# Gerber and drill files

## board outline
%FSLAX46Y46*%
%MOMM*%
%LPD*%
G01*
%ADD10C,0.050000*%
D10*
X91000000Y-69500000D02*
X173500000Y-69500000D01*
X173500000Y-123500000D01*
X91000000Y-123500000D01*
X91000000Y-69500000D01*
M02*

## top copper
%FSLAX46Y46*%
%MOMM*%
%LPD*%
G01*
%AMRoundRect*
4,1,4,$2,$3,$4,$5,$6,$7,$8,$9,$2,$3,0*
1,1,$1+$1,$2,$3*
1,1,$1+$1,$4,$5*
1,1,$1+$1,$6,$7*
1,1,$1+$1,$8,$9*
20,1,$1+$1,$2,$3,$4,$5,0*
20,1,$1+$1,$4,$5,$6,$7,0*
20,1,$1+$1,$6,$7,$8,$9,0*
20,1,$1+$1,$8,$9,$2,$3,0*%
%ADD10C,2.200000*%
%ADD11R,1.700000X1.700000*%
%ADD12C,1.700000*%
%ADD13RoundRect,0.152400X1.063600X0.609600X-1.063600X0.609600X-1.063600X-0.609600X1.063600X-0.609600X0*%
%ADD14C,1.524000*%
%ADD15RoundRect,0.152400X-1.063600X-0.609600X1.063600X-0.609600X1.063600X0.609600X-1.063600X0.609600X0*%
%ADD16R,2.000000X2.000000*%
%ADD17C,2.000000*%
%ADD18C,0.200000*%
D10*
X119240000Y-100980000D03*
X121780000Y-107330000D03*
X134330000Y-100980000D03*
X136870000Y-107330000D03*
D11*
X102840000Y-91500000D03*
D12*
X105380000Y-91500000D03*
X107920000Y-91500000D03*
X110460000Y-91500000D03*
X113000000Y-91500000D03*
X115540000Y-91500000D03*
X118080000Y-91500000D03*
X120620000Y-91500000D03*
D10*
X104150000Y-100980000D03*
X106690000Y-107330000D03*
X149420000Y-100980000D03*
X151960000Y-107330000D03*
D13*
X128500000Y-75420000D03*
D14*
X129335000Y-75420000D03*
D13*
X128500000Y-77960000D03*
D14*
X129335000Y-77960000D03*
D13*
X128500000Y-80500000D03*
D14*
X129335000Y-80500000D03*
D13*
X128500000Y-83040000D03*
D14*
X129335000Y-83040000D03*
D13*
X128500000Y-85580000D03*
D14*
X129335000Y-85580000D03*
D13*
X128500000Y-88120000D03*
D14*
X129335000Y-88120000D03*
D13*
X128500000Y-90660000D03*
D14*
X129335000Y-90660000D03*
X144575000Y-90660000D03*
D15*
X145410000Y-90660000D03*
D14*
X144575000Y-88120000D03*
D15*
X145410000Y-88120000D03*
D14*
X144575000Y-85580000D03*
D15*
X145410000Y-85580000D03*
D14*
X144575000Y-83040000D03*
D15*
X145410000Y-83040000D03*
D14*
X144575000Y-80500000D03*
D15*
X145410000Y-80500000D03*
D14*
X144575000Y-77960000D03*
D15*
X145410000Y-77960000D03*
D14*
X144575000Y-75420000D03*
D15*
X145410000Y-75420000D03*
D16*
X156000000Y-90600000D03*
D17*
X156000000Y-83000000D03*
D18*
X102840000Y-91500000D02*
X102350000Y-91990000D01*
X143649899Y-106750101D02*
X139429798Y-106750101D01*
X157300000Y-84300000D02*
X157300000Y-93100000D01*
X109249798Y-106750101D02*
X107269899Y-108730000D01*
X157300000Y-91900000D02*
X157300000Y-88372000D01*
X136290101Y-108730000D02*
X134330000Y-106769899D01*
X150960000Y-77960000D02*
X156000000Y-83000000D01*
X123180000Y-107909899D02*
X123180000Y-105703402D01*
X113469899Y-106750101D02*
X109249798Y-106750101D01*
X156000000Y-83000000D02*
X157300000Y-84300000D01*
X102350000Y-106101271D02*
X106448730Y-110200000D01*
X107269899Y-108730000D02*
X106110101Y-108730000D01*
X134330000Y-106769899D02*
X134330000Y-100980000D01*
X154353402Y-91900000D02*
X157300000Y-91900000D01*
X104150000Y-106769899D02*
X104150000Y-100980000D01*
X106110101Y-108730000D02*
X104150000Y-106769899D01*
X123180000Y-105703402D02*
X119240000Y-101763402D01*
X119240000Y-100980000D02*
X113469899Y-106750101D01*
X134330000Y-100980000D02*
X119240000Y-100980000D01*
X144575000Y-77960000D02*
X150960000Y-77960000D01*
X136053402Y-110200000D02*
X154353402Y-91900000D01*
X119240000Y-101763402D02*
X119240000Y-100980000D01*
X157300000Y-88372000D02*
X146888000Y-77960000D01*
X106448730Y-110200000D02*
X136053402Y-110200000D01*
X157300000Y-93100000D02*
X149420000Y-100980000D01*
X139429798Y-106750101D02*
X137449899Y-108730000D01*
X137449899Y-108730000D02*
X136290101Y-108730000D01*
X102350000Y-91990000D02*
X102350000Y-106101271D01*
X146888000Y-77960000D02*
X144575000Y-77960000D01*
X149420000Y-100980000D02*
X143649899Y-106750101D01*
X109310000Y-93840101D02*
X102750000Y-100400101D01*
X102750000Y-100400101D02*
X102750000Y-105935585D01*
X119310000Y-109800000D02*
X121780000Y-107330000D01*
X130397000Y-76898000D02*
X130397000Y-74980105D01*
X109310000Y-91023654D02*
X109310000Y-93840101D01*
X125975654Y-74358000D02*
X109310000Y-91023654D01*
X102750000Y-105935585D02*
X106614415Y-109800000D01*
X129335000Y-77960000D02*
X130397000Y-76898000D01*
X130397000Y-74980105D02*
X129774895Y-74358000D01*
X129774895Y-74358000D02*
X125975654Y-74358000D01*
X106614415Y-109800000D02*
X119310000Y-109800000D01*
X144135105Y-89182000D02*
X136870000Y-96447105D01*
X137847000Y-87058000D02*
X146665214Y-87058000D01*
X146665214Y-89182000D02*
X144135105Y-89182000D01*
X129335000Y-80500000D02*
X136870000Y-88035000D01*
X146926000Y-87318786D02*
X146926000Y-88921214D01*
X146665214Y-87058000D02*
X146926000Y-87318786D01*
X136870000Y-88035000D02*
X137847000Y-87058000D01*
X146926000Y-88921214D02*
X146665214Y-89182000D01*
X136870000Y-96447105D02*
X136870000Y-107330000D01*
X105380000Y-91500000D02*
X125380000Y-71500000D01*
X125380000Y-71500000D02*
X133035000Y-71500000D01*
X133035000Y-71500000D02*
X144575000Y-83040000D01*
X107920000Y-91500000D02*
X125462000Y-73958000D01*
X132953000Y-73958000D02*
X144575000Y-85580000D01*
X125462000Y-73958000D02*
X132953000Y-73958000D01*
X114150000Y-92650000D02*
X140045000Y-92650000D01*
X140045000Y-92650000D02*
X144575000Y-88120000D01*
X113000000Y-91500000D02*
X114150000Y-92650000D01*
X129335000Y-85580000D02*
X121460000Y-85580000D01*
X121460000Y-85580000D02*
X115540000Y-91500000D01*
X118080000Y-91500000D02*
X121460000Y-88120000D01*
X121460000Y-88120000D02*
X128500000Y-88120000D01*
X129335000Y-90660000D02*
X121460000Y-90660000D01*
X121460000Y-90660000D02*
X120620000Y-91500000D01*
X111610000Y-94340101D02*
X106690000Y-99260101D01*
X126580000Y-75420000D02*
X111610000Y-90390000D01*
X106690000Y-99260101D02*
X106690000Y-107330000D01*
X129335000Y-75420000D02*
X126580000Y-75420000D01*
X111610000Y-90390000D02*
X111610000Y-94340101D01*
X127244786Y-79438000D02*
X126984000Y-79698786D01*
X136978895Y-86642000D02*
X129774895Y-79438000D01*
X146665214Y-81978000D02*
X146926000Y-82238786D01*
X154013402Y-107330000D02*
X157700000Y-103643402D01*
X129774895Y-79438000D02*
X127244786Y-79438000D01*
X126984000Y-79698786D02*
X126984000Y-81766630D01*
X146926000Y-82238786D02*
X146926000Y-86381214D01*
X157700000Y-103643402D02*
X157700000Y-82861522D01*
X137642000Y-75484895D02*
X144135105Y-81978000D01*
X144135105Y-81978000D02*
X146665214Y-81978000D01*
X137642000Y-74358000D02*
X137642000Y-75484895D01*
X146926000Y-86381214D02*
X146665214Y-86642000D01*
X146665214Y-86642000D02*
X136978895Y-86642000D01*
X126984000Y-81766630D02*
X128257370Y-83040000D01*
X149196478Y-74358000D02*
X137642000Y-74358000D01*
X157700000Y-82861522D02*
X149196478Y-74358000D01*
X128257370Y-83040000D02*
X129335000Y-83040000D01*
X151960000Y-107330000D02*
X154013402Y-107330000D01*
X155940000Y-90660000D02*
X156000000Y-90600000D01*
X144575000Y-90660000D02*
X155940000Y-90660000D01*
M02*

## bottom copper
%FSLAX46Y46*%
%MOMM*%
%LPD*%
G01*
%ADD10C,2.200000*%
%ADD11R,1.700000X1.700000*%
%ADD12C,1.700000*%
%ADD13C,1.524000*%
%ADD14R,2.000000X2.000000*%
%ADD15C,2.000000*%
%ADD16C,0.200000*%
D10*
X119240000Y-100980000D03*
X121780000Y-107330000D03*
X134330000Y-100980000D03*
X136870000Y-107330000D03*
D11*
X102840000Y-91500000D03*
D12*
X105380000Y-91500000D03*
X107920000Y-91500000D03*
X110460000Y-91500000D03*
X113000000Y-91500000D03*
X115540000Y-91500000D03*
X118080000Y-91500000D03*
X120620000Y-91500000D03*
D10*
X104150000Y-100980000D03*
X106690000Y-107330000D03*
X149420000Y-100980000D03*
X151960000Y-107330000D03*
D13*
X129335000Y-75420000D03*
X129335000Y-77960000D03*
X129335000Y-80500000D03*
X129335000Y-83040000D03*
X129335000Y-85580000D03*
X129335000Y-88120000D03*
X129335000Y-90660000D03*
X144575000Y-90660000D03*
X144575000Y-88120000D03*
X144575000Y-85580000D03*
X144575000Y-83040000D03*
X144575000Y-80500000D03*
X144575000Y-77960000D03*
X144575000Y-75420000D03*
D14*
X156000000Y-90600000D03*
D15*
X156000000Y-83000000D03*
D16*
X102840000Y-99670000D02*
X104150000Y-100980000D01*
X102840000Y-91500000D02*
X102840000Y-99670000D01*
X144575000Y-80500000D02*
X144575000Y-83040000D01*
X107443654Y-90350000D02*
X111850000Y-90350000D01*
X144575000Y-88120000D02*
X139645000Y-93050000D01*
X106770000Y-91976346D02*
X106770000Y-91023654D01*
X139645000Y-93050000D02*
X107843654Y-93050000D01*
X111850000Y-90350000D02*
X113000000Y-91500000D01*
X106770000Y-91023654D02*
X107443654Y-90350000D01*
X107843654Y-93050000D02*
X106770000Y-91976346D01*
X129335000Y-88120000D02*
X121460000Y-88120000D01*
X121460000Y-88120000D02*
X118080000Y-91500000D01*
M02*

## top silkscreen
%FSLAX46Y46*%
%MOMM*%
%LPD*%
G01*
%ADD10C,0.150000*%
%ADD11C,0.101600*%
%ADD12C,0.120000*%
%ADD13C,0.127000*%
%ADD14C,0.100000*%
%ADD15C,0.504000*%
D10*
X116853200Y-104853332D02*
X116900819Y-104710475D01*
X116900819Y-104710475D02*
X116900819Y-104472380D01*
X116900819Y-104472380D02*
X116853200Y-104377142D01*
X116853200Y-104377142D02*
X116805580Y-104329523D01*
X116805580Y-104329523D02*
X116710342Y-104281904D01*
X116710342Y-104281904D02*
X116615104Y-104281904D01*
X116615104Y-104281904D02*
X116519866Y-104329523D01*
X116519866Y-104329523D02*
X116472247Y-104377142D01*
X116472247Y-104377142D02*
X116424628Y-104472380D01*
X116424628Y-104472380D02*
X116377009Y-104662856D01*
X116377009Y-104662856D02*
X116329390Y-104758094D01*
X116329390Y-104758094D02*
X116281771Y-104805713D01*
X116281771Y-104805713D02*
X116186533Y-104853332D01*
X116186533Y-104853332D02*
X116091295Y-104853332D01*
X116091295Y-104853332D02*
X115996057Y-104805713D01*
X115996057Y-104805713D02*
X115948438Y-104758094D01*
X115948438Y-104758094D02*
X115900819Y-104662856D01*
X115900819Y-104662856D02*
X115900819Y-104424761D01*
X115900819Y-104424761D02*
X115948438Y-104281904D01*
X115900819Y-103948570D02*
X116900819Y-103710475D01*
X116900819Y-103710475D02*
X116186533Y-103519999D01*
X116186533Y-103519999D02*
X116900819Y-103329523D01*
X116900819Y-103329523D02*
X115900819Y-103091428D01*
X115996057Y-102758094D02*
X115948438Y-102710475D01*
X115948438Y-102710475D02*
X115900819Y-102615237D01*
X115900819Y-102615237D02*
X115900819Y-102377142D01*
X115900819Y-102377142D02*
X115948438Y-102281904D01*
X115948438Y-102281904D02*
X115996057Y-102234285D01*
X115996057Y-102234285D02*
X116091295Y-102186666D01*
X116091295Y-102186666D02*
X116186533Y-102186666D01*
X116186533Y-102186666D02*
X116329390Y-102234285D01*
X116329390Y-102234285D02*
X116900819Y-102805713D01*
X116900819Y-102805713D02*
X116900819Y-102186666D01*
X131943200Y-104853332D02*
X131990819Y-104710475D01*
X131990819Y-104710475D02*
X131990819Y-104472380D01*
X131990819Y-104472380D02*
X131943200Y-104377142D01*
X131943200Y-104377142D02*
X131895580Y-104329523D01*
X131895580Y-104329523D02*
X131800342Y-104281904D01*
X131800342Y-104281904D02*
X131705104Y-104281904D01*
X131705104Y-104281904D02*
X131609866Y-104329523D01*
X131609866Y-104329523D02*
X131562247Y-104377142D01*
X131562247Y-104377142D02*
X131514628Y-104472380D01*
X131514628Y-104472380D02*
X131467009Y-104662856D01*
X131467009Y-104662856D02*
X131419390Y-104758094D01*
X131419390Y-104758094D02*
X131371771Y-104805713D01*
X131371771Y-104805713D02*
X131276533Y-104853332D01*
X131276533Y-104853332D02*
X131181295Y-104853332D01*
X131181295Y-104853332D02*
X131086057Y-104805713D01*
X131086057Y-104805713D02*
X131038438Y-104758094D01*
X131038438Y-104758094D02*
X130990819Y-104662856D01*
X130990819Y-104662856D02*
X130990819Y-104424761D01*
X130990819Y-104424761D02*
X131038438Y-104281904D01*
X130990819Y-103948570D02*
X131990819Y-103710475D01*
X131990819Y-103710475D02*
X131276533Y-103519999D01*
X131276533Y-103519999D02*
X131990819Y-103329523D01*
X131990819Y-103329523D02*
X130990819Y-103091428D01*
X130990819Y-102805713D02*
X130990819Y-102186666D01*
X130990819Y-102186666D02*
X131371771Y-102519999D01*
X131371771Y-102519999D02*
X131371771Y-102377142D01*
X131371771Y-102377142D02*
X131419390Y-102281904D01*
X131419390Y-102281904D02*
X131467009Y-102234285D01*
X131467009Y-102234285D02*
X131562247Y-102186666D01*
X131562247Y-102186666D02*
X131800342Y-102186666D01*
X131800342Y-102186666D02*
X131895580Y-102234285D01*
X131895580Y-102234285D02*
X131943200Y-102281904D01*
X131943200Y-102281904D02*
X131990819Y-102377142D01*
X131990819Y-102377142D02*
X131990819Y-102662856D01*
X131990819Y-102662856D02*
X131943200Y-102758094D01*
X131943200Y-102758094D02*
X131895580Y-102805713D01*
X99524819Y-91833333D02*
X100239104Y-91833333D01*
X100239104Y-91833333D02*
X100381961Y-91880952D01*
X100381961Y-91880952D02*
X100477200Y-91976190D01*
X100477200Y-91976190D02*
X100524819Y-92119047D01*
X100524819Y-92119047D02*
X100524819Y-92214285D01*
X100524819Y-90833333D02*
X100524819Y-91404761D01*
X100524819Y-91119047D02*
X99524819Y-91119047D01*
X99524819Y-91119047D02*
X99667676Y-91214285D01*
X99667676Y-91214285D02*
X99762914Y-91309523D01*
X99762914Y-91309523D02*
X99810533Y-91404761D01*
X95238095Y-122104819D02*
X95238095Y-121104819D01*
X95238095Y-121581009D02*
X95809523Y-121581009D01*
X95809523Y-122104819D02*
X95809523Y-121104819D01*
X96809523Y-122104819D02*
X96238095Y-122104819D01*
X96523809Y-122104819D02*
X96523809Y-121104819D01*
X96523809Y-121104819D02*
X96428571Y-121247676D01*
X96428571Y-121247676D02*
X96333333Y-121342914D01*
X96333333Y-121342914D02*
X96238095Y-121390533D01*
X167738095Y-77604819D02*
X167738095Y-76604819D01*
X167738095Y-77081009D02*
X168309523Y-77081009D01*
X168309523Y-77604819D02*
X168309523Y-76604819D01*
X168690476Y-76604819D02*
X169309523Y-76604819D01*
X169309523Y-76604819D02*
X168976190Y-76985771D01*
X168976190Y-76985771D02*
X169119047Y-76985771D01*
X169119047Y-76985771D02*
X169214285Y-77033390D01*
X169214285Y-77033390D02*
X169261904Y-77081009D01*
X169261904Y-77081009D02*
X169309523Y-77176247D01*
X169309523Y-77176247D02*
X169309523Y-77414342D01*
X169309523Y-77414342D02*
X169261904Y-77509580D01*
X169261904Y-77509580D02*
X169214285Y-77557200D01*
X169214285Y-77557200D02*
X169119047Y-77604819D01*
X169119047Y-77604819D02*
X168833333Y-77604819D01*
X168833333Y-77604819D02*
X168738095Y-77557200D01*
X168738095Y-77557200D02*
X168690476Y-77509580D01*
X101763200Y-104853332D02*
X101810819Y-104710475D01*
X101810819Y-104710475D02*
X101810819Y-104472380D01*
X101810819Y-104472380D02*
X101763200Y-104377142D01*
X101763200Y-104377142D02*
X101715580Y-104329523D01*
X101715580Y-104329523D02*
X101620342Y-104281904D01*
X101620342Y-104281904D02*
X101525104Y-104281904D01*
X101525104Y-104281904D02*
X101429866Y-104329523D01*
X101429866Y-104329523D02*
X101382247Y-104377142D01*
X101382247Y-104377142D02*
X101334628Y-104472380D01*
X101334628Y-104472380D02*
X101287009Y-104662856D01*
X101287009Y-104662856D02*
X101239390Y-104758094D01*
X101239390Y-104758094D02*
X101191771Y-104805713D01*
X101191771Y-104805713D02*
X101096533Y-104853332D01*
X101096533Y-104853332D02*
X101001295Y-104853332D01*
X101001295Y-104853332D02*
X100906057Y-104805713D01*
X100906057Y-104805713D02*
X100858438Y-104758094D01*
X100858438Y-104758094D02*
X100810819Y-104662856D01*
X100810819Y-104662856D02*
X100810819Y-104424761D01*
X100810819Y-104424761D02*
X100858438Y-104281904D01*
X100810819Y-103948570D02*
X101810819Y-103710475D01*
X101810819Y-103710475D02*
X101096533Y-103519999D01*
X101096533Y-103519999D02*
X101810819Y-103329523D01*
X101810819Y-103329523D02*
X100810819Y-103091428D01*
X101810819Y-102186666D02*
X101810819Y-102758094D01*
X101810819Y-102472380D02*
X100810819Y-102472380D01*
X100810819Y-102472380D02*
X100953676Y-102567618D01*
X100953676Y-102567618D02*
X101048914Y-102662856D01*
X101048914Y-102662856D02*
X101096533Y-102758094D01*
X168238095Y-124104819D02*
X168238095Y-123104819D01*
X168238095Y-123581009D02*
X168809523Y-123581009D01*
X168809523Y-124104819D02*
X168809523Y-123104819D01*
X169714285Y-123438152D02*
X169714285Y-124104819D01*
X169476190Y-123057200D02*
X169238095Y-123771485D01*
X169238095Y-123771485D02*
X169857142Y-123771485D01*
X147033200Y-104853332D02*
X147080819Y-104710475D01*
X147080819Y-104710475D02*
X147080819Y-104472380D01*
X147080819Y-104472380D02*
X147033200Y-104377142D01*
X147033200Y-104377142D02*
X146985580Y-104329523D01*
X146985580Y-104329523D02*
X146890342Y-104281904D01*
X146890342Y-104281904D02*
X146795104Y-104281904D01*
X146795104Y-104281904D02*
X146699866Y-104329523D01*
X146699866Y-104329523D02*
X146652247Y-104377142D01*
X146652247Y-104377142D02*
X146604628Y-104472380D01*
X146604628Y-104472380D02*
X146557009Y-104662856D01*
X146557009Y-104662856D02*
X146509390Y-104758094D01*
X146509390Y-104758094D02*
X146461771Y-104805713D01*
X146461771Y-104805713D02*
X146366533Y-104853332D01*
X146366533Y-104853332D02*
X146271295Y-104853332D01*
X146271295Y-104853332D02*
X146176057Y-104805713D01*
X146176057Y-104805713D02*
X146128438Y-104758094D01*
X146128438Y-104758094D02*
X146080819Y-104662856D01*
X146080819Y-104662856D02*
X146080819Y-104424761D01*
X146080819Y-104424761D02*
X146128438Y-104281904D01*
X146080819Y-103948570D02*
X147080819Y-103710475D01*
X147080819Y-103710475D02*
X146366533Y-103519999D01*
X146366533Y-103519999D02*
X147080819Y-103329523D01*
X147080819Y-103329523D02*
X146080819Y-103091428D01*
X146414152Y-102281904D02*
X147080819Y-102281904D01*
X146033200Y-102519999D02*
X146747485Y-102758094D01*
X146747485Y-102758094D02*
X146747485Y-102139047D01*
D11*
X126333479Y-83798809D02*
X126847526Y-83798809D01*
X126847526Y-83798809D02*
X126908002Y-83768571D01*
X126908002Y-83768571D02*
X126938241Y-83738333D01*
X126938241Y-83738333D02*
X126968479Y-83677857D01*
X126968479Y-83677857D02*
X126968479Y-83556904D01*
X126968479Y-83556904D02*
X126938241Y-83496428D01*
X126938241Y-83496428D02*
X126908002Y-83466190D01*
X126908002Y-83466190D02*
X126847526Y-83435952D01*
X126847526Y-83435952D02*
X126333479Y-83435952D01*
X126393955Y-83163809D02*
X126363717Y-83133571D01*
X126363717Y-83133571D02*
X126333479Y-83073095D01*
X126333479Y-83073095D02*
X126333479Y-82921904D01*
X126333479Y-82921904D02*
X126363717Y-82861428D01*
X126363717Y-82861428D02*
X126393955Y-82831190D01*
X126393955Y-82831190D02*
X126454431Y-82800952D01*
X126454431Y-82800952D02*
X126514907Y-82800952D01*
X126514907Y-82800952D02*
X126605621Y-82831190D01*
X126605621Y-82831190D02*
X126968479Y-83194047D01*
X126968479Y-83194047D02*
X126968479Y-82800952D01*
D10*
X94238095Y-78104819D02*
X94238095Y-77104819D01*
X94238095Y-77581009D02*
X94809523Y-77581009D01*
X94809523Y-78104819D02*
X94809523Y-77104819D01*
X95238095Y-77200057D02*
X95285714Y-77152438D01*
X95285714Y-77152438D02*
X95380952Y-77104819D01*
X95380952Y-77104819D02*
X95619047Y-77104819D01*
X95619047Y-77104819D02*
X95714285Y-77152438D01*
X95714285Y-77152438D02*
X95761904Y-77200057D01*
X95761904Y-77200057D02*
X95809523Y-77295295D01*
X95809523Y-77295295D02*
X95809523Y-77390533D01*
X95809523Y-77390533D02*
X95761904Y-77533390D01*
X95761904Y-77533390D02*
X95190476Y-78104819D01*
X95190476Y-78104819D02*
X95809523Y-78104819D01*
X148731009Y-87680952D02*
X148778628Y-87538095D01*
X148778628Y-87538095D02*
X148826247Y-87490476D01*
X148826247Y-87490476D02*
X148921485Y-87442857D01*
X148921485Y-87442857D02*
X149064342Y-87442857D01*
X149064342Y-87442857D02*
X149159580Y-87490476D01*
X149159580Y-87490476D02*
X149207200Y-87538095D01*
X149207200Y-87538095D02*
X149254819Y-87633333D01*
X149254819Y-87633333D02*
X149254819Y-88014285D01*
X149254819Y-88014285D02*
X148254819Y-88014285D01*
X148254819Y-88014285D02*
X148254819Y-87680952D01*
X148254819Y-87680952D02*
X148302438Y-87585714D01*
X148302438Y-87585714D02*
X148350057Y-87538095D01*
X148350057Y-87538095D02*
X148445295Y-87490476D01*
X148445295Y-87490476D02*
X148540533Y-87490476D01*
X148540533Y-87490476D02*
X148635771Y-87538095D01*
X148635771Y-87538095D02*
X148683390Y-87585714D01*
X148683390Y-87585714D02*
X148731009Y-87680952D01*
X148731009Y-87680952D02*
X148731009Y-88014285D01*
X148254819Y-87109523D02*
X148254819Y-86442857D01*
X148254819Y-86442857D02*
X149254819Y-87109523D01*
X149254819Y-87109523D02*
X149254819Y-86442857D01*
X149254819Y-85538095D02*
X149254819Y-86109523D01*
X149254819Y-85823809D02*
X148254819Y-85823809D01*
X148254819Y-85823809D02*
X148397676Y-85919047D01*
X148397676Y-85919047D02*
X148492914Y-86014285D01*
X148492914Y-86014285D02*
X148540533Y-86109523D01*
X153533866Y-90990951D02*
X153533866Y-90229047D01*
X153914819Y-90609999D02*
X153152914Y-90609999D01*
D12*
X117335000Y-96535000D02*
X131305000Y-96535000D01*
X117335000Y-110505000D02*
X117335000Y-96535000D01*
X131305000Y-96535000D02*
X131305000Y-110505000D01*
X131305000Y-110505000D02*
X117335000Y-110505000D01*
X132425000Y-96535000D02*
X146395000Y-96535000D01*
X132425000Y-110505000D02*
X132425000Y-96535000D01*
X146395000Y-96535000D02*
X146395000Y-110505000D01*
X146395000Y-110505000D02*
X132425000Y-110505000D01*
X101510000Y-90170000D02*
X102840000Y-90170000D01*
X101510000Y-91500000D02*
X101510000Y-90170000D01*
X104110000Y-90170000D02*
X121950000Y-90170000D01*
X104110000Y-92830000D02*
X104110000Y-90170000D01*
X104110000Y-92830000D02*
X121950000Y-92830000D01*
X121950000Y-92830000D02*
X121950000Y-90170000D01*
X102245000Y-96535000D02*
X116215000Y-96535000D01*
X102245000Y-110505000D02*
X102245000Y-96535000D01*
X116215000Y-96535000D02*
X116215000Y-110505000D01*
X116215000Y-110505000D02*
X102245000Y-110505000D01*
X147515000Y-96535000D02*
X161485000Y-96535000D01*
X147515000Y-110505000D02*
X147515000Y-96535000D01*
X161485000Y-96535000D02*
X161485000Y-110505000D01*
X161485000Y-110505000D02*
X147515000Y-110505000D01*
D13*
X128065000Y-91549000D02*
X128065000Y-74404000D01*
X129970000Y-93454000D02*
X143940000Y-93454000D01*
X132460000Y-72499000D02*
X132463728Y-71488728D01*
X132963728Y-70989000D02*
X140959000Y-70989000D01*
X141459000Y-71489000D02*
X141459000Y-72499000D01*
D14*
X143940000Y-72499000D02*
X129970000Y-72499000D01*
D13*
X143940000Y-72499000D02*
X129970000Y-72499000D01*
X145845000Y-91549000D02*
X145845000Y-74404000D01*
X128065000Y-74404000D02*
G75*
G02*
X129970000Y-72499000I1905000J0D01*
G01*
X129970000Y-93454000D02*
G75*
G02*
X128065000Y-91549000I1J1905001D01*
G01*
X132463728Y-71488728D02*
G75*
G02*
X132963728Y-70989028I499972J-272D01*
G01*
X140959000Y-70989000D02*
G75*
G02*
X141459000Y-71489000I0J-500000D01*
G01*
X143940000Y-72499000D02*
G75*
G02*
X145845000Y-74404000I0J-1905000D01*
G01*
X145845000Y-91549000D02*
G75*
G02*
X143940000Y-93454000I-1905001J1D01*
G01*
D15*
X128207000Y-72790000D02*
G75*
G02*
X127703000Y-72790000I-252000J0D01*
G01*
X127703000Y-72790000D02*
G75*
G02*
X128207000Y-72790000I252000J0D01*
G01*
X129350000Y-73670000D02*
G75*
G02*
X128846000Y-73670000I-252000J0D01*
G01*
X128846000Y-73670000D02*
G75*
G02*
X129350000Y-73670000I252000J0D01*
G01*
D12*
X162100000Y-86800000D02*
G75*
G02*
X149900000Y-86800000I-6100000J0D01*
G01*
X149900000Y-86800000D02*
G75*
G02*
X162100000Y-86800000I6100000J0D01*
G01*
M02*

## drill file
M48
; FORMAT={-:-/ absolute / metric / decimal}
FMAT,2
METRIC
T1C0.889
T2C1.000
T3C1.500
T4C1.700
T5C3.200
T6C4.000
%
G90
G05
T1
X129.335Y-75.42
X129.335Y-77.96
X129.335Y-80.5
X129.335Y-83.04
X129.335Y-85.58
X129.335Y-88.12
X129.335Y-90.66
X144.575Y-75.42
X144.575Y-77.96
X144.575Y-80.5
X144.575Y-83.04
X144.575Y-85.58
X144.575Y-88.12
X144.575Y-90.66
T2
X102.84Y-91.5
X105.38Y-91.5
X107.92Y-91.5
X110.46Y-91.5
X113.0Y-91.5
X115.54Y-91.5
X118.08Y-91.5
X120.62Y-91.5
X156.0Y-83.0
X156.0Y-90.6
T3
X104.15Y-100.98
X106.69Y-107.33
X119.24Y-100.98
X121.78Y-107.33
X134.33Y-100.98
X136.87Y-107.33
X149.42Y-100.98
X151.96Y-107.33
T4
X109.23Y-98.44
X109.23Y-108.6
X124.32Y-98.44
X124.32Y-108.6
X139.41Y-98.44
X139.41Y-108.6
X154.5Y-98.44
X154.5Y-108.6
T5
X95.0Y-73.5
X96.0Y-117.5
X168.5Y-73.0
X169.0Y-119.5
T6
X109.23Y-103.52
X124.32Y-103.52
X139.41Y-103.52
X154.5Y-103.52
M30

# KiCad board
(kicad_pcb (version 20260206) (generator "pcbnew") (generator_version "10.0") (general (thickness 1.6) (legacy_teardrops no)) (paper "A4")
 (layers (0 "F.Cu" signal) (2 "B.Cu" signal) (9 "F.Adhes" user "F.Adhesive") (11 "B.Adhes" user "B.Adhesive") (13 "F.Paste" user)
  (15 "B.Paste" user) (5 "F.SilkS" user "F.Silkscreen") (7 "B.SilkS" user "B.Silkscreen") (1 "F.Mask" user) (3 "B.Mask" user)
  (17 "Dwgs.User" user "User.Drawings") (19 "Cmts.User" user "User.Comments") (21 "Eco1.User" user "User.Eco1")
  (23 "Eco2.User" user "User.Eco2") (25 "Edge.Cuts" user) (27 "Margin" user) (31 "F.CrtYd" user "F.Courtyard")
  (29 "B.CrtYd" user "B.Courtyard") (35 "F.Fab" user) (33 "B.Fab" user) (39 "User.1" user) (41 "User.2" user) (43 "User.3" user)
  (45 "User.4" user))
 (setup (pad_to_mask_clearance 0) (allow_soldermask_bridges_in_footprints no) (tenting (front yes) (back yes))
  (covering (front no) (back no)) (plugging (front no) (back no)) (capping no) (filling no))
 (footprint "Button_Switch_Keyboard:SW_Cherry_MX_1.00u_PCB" (layer "F.Cu") (at 119.24 100.98 90)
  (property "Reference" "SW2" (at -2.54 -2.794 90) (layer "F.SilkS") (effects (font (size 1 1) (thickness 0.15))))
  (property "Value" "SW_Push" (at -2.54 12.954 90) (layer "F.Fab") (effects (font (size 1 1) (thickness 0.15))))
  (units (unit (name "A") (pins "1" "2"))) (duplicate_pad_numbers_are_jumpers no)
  (fp_line (start 4.445 -1.905) (end 4.445 12.065) (stroke (width 0.12) (type solid)) (layer "F.SilkS"))
  (fp_line (start -9.525 -1.905) (end 4.445 -1.905) (stroke (width 0.12) (type solid)) (layer "F.SilkS"))
  (fp_line (start 4.445 12.065) (end -9.525 12.065) (stroke (width 0.12) (type solid)) (layer "F.SilkS"))
  (fp_line (start -9.525 12.065) (end -9.525 -1.905) (stroke (width 0.12) (type solid)) (layer "F.SilkS"))
  (pad "" np_thru_hole circle (at -7.62 5.08 90) (size 1.7 1.7) (drill 1.7) (layers "*.Cu" "*.Mask"))
  (pad "" np_thru_hole circle (at -2.54 5.08 90) (size 4 4) (drill 4) (layers "*.Cu" "*.Mask"))
  (pad "" np_thru_hole circle (at 2.54 5.08 90) (size 1.7 1.7) (drill 1.7) (layers "*.Cu" "*.Mask"))
  (pad "1" thru_hole circle (at 0 0 90) (size 2.2 2.2) (drill 1.5) (layers "*.Cu" "*.Mask") (remove_unused_layers no) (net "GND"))
  (pad "2" thru_hole circle (at -6.35 2.54 90) (size 2.2 2.2) (drill 1.5) (layers "*.Cu" "*.Mask") (remove_unused_layers no)
   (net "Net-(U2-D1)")))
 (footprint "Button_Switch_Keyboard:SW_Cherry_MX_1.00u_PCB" (layer "F.Cu") (at 134.33 100.98 90)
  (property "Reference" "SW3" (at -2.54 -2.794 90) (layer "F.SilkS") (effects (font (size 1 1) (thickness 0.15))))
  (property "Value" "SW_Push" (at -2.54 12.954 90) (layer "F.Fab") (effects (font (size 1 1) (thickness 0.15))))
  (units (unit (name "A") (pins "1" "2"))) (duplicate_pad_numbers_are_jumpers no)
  (fp_line (start 4.445 -1.905) (end 4.445 12.065) (stroke (width 0.12) (type solid)) (layer "F.SilkS"))
  (fp_line (start -9.525 -1.905) (end 4.445 -1.905) (stroke (width 0.12) (type solid)) (layer "F.SilkS"))
  (fp_line (start 4.445 12.065) (end -9.525 12.065) (stroke (width 0.12) (type solid)) (layer "F.SilkS"))
  (fp_line (start -9.525 12.065) (end -9.525 -1.905) (stroke (width 0.12) (type solid)) (layer "F.SilkS"))
  (pad "" np_thru_hole circle (at -7.62 5.08 90) (size 1.7 1.7) (drill 1.7) (layers "*.Cu" "*.Mask"))
  (pad "" np_thru_hole circle (at -2.54 5.08 90) (size 4 4) (drill 4) (layers "*.Cu" "*.Mask"))
  (pad "" np_thru_hole circle (at 2.54 5.08 90) (size 1.7 1.7) (drill 1.7) (layers "*.Cu" "*.Mask"))
  (pad "1" thru_hole circle (at 0 0 90) (size 2.2 2.2) (drill 1.5) (layers "*.Cu" "*.Mask") (remove_unused_layers no) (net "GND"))
  (pad "2" thru_hole circle (at -6.35 2.54 90) (size 2.2 2.2) (drill 1.5) (layers "*.Cu" "*.Mask") (remove_unused_layers no)
   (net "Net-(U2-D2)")))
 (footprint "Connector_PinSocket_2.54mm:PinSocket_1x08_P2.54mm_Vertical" (layer "F.Cu") (at 102.84 91.5 90)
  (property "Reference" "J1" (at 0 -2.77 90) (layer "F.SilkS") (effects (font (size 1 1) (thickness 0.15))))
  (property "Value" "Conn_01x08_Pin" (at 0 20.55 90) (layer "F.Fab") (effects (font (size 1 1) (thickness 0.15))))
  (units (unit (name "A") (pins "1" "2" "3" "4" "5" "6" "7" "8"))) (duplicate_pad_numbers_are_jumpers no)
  (fp_line (start 1.33 -1.33) (end 1.33 0) (stroke (width 0.12) (type solid)) (layer "F.SilkS"))
  (fp_line (start 0 -1.33) (end 1.33 -1.33) (stroke (width 0.12) (type solid)) (layer "F.SilkS"))
  (fp_line (start 1.33 1.27) (end 1.33 19.11) (stroke (width 0.12) (type solid)) (layer "F.SilkS"))
  (fp_line (start -1.33 1.27) (end 1.33 1.27) (stroke (width 0.12) (type solid)) (layer "F.SilkS"))
  (fp_line (start -1.33 1.27) (end -1.33 19.11) (stroke (width 0.12) (type solid)) (layer "F.SilkS"))
  (fp_line (start -1.33 19.11) (end 1.33 19.11) (stroke (width 0.12) (type solid)) (layer "F.SilkS"))
  (pad "1" thru_hole rect (at 0 0 90) (size 1.7 1.7) (drill 1) (layers "*.Cu" "*.Mask") (remove_unused_layers no) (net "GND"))
  (pad "2" thru_hole circle (at 0 2.54 90) (size 1.7 1.7) (drill 1) (layers "*.Cu" "*.Mask") (remove_unused_layers no) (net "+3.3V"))
  (pad "3" thru_hole circle (at 0 5.08 90) (size 1.7 1.7) (drill 1) (layers "*.Cu" "*.Mask") (remove_unused_layers no) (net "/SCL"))
  (pad "4" thru_hole circle (at 0 7.62 90) (size 1.7 1.7) (drill 1) (layers "*.Cu" "*.Mask") (remove_unused_layers no) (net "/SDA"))
  (pad "5" thru_hole circle (at 0 10.16 90) (size 1.7 1.7) (drill 1) (layers "*.Cu" "*.Mask") (remove_unused_layers no) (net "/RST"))
  (pad "6" thru_hole circle (at 0 12.7 90) (size 1.7 1.7) (drill 1) (layers "*.Cu" "*.Mask") (remove_unused_layers no) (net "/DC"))
  (pad "7" thru_hole circle (at 0 15.24 90) (size 1.7 1.7) (drill 1) (layers "*.Cu" "*.Mask") (remove_unused_layers no) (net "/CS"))
  (pad "8" thru_hole circle (at 0 17.78 90) (size 1.7 1.7) (drill 1) (layers "*.Cu" "*.Mask") (remove_unused_layers no) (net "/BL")))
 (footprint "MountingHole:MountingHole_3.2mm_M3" (layer "F.Cu") (at 96 117.5 180)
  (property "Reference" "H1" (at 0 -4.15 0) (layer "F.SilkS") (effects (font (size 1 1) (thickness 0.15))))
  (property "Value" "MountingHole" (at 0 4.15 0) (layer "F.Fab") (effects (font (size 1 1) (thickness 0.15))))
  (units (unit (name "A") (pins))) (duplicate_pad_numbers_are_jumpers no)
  (pad "" np_thru_hole circle (at 0 0 180) (size 3.2 3.2) (drill 3.2) (layers "*.Cu" "*.Mask")))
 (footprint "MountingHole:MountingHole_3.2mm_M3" (layer "F.Cu") (at 168.5 73 180)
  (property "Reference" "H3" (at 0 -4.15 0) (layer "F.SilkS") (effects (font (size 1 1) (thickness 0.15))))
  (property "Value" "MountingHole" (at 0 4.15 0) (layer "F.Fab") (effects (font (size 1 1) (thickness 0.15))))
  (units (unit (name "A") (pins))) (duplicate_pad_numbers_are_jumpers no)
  (pad "" np_thru_hole circle (at 0 0 180) (size 3.2 3.2) (drill 3.2) (layers "*.Cu" "*.Mask")))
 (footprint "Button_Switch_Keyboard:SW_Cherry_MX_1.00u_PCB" (layer "F.Cu") (at 104.15 100.98 90)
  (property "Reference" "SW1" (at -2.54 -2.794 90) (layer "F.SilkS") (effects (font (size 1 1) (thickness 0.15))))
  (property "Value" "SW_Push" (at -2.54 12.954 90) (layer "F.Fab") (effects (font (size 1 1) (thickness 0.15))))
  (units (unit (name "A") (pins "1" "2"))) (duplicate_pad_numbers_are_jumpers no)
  (fp_line (start 4.445 -1.905) (end 4.445 12.065) (stroke (width 0.12) (type solid)) (layer "F.SilkS"))
  (fp_line (start -9.525 -1.905) (end 4.445 -1.905) (stroke (width 0.12) (type solid)) (layer "F.SilkS"))
  (fp_line (start 4.445 12.065) (end -9.525 12.065) (stroke (width 0.12) (type solid)) (layer "F.SilkS"))
  (fp_line (start -9.525 12.065) (end -9.525 -1.905) (stroke (width 0.12) (type solid)) (layer "F.SilkS"))
  (pad "" np_thru_hole circle (at -7.62 5.08 90) (size 1.7 1.7) (drill 1.7) (layers "*.Cu" "*.Mask"))
  (pad "" np_thru_hole circle (at -2.54 5.08 90) (size 4 4) (drill 4) (layers "*.Cu" "*.Mask"))
  (pad "" np_thru_hole circle (at 2.54 5.08 90) (size 1.7 1.7) (drill 1.7) (layers "*.Cu" "*.Mask"))
  (pad "1" thru_hole circle (at 0 0 90) (size 2.2 2.2) (drill 1.5) (layers "*.Cu" "*.Mask") (remove_unused_layers no) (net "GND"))
  (pad "2" thru_hole circle (at -6.35 2.54 90) (size 2.2 2.2) (drill 1.5) (layers "*.Cu" "*.Mask") (remove_unused_layers no)
   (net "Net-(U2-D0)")))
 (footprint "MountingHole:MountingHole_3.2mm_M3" (layer "F.Cu") (at 169 119.5 180)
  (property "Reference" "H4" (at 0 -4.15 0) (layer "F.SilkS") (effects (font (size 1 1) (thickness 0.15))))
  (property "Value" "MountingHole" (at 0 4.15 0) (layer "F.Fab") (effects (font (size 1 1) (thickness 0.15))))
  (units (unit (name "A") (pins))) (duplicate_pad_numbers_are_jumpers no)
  (pad "" np_thru_hole circle (at 0 0 180) (size 3.2 3.2) (drill 3.2) (layers "*.Cu" "*.Mask")))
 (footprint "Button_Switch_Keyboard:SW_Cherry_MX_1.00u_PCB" (layer "F.Cu") (at 149.42 100.98 90)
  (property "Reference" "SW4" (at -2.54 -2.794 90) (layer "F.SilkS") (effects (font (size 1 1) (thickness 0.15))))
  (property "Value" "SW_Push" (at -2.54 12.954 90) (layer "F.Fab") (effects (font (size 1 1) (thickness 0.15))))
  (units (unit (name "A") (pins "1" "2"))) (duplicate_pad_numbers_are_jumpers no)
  (fp_line (start 4.445 -1.905) (end 4.445 12.065) (stroke (width 0.12) (type solid)) (layer "F.SilkS"))
  (fp_line (start -9.525 -1.905) (end 4.445 -1.905) (stroke (width 0.12) (type solid)) (layer "F.SilkS"))
  (fp_line (start 4.445 12.065) (end -9.525 12.065) (stroke (width 0.12) (type solid)) (layer "F.SilkS"))
  (fp_line (start -9.525 12.065) (end -9.525 -1.905) (stroke (width 0.12) (type solid)) (layer "F.SilkS"))
  (pad "" np_thru_hole circle (at -7.62 5.08 90) (size 1.7 1.7) (drill 1.7) (layers "*.Cu" "*.Mask"))
  (pad "" np_thru_hole circle (at -2.54 5.08 90) (size 4 4) (drill 4) (layers "*.Cu" "*.Mask"))
  (pad "" np_thru_hole circle (at 2.54 5.08 90) (size 1.7 1.7) (drill 1.7) (layers "*.Cu" "*.Mask"))
  (pad "1" thru_hole circle (at 0 0 90) (size 2.2 2.2) (drill 1.5) (layers "*.Cu" "*.Mask") (remove_unused_layers no) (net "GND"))
  (pad "2" thru_hole circle (at -6.35 2.54 90) (size 2.2 2.2) (drill 1.5) (layers "*.Cu" "*.Mask") (remove_unused_layers no)
   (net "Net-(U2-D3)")))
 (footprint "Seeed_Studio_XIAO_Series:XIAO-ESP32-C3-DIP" (layer "F.Cu") (at 136.955 83.04 90)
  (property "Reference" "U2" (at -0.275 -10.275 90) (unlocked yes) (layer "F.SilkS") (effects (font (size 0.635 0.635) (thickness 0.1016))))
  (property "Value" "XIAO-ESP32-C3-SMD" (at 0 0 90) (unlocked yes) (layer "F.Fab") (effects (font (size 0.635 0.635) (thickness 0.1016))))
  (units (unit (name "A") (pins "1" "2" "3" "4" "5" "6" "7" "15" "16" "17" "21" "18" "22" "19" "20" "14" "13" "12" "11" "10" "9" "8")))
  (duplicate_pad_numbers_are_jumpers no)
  (fp_line (start -8.509 -8.89) (end 8.636 -8.89) (stroke (width 0.127) (type solid)) (layer "F.SilkS"))
  (fp_line (start -10.414 -6.985) (end -10.414 6.985) (stroke (width 0.127) (type solid)) (layer "F.SilkS"))
  (fp_line (start 10.541 -4.495) (end 11.551272 -4.491272) (stroke (width 0.127) (type solid)) (layer "F.SilkS"))
  (fp_line (start 12.051 -3.991272) (end 12.051 4.004) (stroke (width 0.127) (type solid)) (layer "F.SilkS"))
  (fp_line (start 11.551 4.504) (end 10.541 4.504) (stroke (width 0.127) (type solid)) (layer "F.SilkS"))
  (fp_line (start 10.541 6.985) (end 10.541 -6.985) (stroke (width 0.1) (type solid)) (layer "F.SilkS"))
  (fp_line (start 10.541 6.985) (end 10.541 -6.985) (stroke (width 0.127) (type solid)) (layer "F.SilkS"))
  (fp_line (start -8.509 8.89) (end 8.636 8.89) (stroke (width 0.127) (type solid)) (layer "F.SilkS"))
  (fp_arc (start 8.636 -8.89) (mid 9.983038 -8.332038) (end 10.541 -6.985) (stroke (width 0.127) (type solid)) (layer "F.SilkS"))
  (fp_arc (start -10.414 -6.985) (mid -9.856038 -8.332038) (end -8.509 -8.89) (stroke (width 0.127) (type solid)) (layer "F.SilkS"))
  (fp_arc (start 11.551272 -4.491272) (mid 11.904644 -4.344724) (end 12.051 -3.991272) (stroke (width 0.127) (type default))
   (layer "F.SilkS"))
  (fp_arc (start 12.051 4.004) (mid 11.904553 4.357553) (end 11.551 4.504) (stroke (width 0.127) (type default)) (layer "F.SilkS"))
  (fp_arc (start 10.541 6.985) (mid 9.983038 8.332038) (end 8.636 8.89) (stroke (width 0.127) (type solid)) (layer "F.SilkS"))
  (fp_arc (start -8.509 8.89) (mid -9.856038 8.332038) (end -10.414 6.985) (stroke (width 0.127) (type solid)) (layer "F.SilkS"))
  (fp_circle (center 10.25 -9) (end 10.504 -9) (stroke (width 0.5) (type solid)) (fill yes) (layer "F.SilkS"))
  (fp_circle (center 9.37 -7.857) (end 9.624 -7.857) (stroke (width 0.5) (type solid)) (fill yes) (layer "F.SilkS"))
  (pad "1" smd roundrect (at 7.62 -8.455 180) (size 2.432 1.524) (layers "F.Cu" "F.Mask") (roundrect_rratio 0.1) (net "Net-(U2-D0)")
   (thermal_bridge_angle 45))
  (pad "1" thru_hole circle (at 7.62 -7.62 180) (size 1.524 1.524) (drill 0.889) (layers "*.Cu" "*.Mask") (remove_unused_layers no)
   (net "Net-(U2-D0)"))
  (pad "2" smd roundrect (at 5.08 -8.455 180) (size 2.432 1.524) (layers "F.Cu" "F.Mask") (roundrect_rratio 0.1) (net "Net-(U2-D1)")
   (thermal_bridge_angle 45))
  (pad "2" thru_hole circle (at 5.08 -7.62 180) (size 1.524 1.524) (drill 0.889) (layers "*.Cu" "*.Mask") (remove_unused_layers no)
   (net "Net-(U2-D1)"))
  (pad "3" smd roundrect (at 2.54 -8.455 180) (size 2.432 1.524) (layers "F.Cu" "F.Mask") (roundrect_rratio 0.1) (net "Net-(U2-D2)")
   (thermal_bridge_angle 45))
  (pad "3" thru_hole circle (at 2.54 -7.62 180) (size 1.524 1.524) (drill 0.889) (layers "*.Cu" "*.Mask") (remove_unused_layers no)
   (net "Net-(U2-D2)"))
  (pad "4" smd roundrect (at 0 -8.455 180) (size 2.432 1.524) (layers "F.Cu" "F.Mask") (roundrect_rratio 0.1) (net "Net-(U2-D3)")
   (thermal_bridge_angle 45))
  (pad "4" thru_hole circle (at 0 -7.62 180) (size 1.524 1.524) (drill 0.889) (layers "*.Cu" "*.Mask") (remove_unused_layers no)
   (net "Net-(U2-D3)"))
  (pad "5" smd roundrect (at -2.54 -8.455 180) (size 2.432 1.524) (layers "F.Cu" "F.Mask") (roundrect_rratio 0.1) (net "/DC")
   (thermal_bridge_angle 45))
  (pad "5" thru_hole circle (at -2.54 -7.62 180) (size 1.524 1.524) (drill 0.889) (layers "*.Cu" "*.Mask") (remove_unused_layers no)
   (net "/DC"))
  (pad "6" smd roundrect (at -5.08 -8.455 180) (size 2.432 1.524) (layers "F.Cu" "F.Mask") (roundrect_rratio 0.1) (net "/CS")
   (thermal_bridge_angle 45))
  (pad "6" thru_hole circle (at -5.08 -7.62 180) (size 1.524 1.524) (drill 0.889) (layers "*.Cu" "*.Mask") (remove_unused_layers no)
   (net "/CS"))
  (pad "7" smd roundrect (at -7.62 -8.455 180) (size 2.432 1.524) (layers "F.Cu" "F.Mask") (roundrect_rratio 0.1) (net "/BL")
   (thermal_bridge_angle 45))
  (pad "7" thru_hole circle (at -7.62 -7.62 180) (size 1.524 1.524) (drill 0.889) (layers "*.Cu" "*.Mask") (remove_unused_layers no)
   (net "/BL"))
  (pad "8" thru_hole circle (at -7.62 7.62) (size 1.524 1.524) (drill 0.889) (layers "*.Cu" "*.Mask") (remove_unused_layers no)
   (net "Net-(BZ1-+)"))
  (pad "8" smd roundrect (at -7.62 8.455) (size 2.432 1.524) (layers "F.Cu" "F.Mask") (roundrect_rratio 0.1) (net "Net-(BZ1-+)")
   (thermal_bridge_angle 45))
  (pad "9" thru_hole circle (at -5.08 7.62) (size 1.524 1.524) (drill 0.889) (layers "*.Cu" "*.Mask") (remove_unused_layers no) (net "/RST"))
  (pad "9" smd roundrect (at -5.08 8.455) (size 2.432 1.524) (layers "F.Cu" "F.Mask") (roundrect_rratio 0.1) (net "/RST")
   (thermal_bridge_angle 45))
  (pad "10" thru_hole circle (at -2.54 7.62) (size 1.524 1.524) (drill 0.889) (layers "*.Cu" "*.Mask") (remove_unused_layers no)
   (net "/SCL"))
  (pad "10" smd roundrect (at -2.54 8.455) (size 2.432 1.524) (layers "F.Cu" "F.Mask") (roundrect_rratio 0.1) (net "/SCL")
   (thermal_bridge_angle 45))
  (pad "11" thru_hole circle (at 0 7.62) (size 1.524 1.524) (drill 0.889) (layers "*.Cu" "*.Mask") (remove_unused_layers no) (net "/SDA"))
  (pad "11" smd roundrect (at 0 8.455) (size 2.432 1.524) (layers "F.Cu" "F.Mask") (roundrect_rratio 0.1) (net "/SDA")
   (thermal_bridge_angle 45))
  (pad "12" thru_hole circle (at 2.54 7.62) (size 1.524 1.524) (drill 0.889) (layers "*.Cu" "*.Mask") (remove_unused_layers no)
   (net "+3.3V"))
  (pad "12" smd roundrect (at 2.54 8.455) (size 2.432 1.524) (layers "F.Cu" "F.Mask") (roundrect_rratio 0.1) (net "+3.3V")
   (thermal_bridge_angle 45))
  (pad "13" thru_hole circle (at 5.08 7.62) (size 1.524 1.524) (drill 0.889) (layers "*.Cu" "*.Mask") (remove_unused_layers no) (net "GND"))
  (pad "13" smd roundrect (at 5.08 8.455) (size 2.432 1.524) (layers "F.Cu" "F.Mask") (roundrect_rratio 0.1) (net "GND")
   (thermal_bridge_angle 45))
  (pad "14" thru_hole circle (at 7.62 7.62) (size 1.524 1.524) (drill 0.889) (layers "*.Cu" "*.Mask") (remove_unused_layers no)
   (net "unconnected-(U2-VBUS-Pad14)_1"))
  (pad "14" smd roundrect (at 7.62 8.455) (size 2.432 1.524) (layers "F.Cu" "F.Mask") (roundrect_rratio 0.1)
   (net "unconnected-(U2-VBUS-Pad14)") (thermal_bridge_angle 45)))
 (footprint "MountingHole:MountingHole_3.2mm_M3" (layer "F.Cu") (at 95 73.5 180)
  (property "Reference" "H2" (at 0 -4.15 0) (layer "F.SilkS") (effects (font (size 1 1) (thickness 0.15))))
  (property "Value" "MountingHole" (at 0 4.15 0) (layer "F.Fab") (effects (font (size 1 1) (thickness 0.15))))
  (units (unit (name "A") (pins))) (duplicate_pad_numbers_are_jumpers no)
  (pad "" np_thru_hole circle (at 0 0 180) (size 3.2 3.2) (drill 3.2) (layers "*.Cu" "*.Mask")))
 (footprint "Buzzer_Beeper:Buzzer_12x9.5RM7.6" (layer "F.Cu") (at 156 90.6 90)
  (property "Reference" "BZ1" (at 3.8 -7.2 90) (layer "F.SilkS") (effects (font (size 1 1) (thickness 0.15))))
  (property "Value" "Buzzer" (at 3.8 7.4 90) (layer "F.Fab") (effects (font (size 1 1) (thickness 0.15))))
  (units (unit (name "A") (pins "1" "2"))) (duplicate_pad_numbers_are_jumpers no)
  (fp_circle (center 3.8 0) (end 9.9 0) (stroke (width 0.12) (type solid)) (fill no) (layer "F.SilkS"))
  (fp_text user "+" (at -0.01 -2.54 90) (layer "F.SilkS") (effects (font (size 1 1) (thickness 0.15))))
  (pad "1" thru_hole rect (at 0 0 90) (size 2 2) (drill 1) (layers "*.Cu" "*.Mask") (remove_unused_layers no) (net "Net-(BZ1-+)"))
  (pad "2" thru_hole circle (at 7.6 0 90) (size 2 2) (drill 1) (layers "*.Cu" "*.Mask") (remove_unused_layers no) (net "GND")))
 (gr_rect (start 91 69.5) (end 173.5 123.5) (stroke (width 0.05) (type default)) (fill no) (layer "Edge.Cuts"))
 (segment (start 102.84 91.5) (end 102.35 91.99) (width 0.2) (layer "F.Cu") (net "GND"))
 (segment (start 143.649899 106.750101) (end 139.429798 106.750101) (width 0.2) (layer "F.Cu") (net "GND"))
 (segment (start 157.3 84.3) (end 157.3 93.1) (width 0.2) (layer "F.Cu") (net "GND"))
 (segment (start 109.249798 106.750101) (end 107.269899 108.73) (width 0.2) (layer "F.Cu") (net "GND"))
 (segment (start 157.3 91.9) (end 157.3 88.372) (width 0.2) (layer "F.Cu") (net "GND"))
 (segment (start 136.290101 108.73) (end 134.33 106.769899) (width 0.2) (layer "F.Cu") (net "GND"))
 (segment (start 150.96 77.96) (end 156 83) (width 0.2) (layer "F.Cu") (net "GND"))
 (segment (start 123.18 107.909899) (end 123.18 105.703402) (width 0.2) (layer "F.Cu") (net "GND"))
 (segment (start 113.469899 106.750101) (end 109.249798 106.750101) (width 0.2) (layer "F.Cu") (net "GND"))
 (segment (start 156 83) (end 157.3 84.3) (width 0.2) (layer "F.Cu") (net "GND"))
 (segment (start 102.35 106.101271) (end 106.44873 110.2) (width 0.2) (layer "F.Cu") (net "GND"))
 (segment (start 107.269899 108.73) (end 106.110101 108.73) (width 0.2) (layer "F.Cu") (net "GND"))
 (segment (start 134.33 106.769899) (end 134.33 100.98) (width 0.2) (layer "F.Cu") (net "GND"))
 (segment (start 154.353402 91.9) (end 157.3 91.9) (width 0.2) (layer "F.Cu") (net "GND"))
 (segment (start 104.15 106.769899) (end 104.15 100.98) (width 0.2) (layer "F.Cu") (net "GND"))
 (segment (start 106.110101 108.73) (end 104.15 106.769899) (width 0.2) (layer "F.Cu") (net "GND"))
 (segment (start 123.18 105.703402) (end 119.24 101.763402) (width 0.2) (layer "F.Cu") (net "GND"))
 (segment (start 119.24 100.98) (end 113.469899 106.750101) (width 0.2) (layer "F.Cu") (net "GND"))
 (segment (start 134.33 100.98) (end 119.24 100.98) (width 0.2) (layer "F.Cu") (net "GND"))
 (segment (start 144.575 77.96) (end 150.96 77.96) (width 0.2) (layer "F.Cu") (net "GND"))
 (segment (start 136.053402 110.2) (end 154.353402 91.9) (width 0.2) (layer "F.Cu") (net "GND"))
 (segment (start 119.24 101.763402) (end 119.24 100.98) (width 0.2) (layer "F.Cu") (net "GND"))
 (segment (start 157.3 88.372) (end 146.888 77.96) (width 0.2) (layer "F.Cu") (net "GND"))
 (segment (start 106.44873 110.2) (end 136.053402 110.2) (width 0.2) (layer "F.Cu") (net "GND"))
 (segment (start 157.3 93.1) (end 149.42 100.98) (width 0.2) (layer "F.Cu") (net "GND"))
 (segment (start 139.429798 106.750101) (end 137.449899 108.73) (width 0.2) (layer "F.Cu") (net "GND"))
 (segment (start 137.449899 108.73) (end 136.290101 108.73) (width 0.2) (layer "F.Cu") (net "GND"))
 (segment (start 102.35 91.99) (end 102.35 106.101271) (width 0.2) (layer "F.Cu") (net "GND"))
 (segment (start 146.888 77.96) (end 144.575 77.96) (width 0.2) (layer "F.Cu") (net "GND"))
 (segment (start 149.42 100.98) (end 143.649899 106.750101) (width 0.2) (layer "F.Cu") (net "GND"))
 (segment (start 102.84 99.67) (end 104.15 100.98) (width 0.2) (layer "B.Cu") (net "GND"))
 (segment (start 102.84 91.5) (end 102.84 99.67) (width 0.2) (layer "B.Cu") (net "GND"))
 (segment (start 109.31 93.840101) (end 102.75 100.400101) (width 0.2) (layer "F.Cu") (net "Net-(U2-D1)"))
 (segment (start 102.75 100.400101) (end 102.75 105.935585) (width 0.2) (layer "F.Cu") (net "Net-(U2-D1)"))
 (segment (start 119.31 109.8) (end 121.78 107.33) (width 0.2) (layer "F.Cu") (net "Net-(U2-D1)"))
 (segment (start 130.397 76.898) (end 130.397 74.980105) (width 0.2) (layer "F.Cu") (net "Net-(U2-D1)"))
 (segment (start 109.31 91.023654) (end 109.31 93.840101) (width 0.2) (layer "F.Cu") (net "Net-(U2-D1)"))
 (segment (start 125.975654 74.358) (end 109.31 91.023654) (width 0.2) (layer "F.Cu") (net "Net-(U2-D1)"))
 (segment (start 102.75 105.935585) (end 106.614415 109.8) (width 0.2) (layer "F.Cu") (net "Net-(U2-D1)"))
 (segment (start 129.335 77.96) (end 130.397 76.898) (width 0.2) (layer "F.Cu") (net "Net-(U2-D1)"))
 (segment (start 130.397 74.980105) (end 129.774895 74.358) (width 0.2) (layer "F.Cu") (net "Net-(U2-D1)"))
 (segment (start 129.774895 74.358) (end 125.975654 74.358) (width 0.2) (layer "F.Cu") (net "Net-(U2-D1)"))
 (segment (start 106.614415 109.8) (end 119.31 109.8) (width 0.2) (layer "F.Cu") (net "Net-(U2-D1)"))
 (segment (start 144.135105 89.182) (end 136.87 96.447105) (width 0.2) (layer "F.Cu") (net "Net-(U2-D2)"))
 (segment (start 137.847 87.058) (end 146.665214 87.058) (width 0.2) (layer "F.Cu") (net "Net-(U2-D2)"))
 (segment (start 146.665214 89.182) (end 144.135105 89.182) (width 0.2) (layer "F.Cu") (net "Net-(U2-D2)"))
 (segment (start 129.335 80.5) (end 136.87 88.035) (width 0.2) (layer "F.Cu") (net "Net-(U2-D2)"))
 (segment (start 146.926 87.318786) (end 146.926 88.921214) (width 0.2) (layer "F.Cu") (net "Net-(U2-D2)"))
 (segment (start 146.665214 87.058) (end 146.926 87.318786) (width 0.2) (layer "F.Cu") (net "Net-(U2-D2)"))
 (segment (start 136.87 88.035) (end 137.847 87.058) (width 0.2) (layer "F.Cu") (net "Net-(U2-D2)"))
 (segment (start 146.926 88.921214) (end 146.665214 89.182) (width 0.2) (layer "F.Cu") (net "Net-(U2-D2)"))
 (segment (start 136.87 96.447105) (end 136.87 107.33) (width 0.2) (layer "F.Cu") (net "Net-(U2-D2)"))
 (segment (start 105.38 91.5) (end 125.38 71.5) (width 0.2) (layer "F.Cu") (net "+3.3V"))
 (segment (start 125.38 71.5) (end 133.035 71.5) (width 0.2) (layer "F.Cu") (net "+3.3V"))
 (segment (start 133.035 71.5) (end 144.575 83.04) (width 0.2) (layer "F.Cu") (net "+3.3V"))
 (segment (start 144.575 80.5) (end 144.575 83.04) (width 0.2) (layer "B.Cu") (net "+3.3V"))
 (segment (start 107.92 91.5) (end 125.462 73.958) (width 0.2) (layer "F.Cu") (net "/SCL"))
 (segment (start 132.953 73.958) (end 144.575 85.58) (width 0.2) (layer "F.Cu") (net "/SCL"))
 (segment (start 125.462 73.958) (end 132.953 73.958) (width 0.2) (layer "F.Cu") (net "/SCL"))
 (segment (start 114.15 92.65) (end 140.045 92.65) (width 0.2) (layer "F.Cu") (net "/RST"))
 (segment (start 140.045 92.65) (end 144.575 88.12) (width 0.2) (layer "F.Cu") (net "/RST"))
 (segment (start 113 91.5) (end 114.15 92.65) (width 0.2) (layer "F.Cu") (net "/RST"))
 (segment (start 107.443654 90.35) (end 111.85 90.35) (width 0.2) (layer "B.Cu") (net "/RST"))
 (segment (start 144.575 88.12) (end 139.645 93.05) (width 0.2) (layer "B.Cu") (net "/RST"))
 (segment (start 106.77 91.976346) (end 106.77 91.023654) (width 0.2) (layer "B.Cu") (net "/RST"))
 (segment (start 139.645 93.05) (end 107.843654 93.05) (width 0.2) (layer "B.Cu") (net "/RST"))
 (segment (start 111.85 90.35) (end 113 91.5) (width 0.2) (layer "B.Cu") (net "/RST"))
 (segment (start 106.77 91.023654) (end 107.443654 90.35) (width 0.2) (layer "B.Cu") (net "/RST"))
 (segment (start 107.843654 93.05) (end 106.77 91.976346) (width 0.2) (layer "B.Cu") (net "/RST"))
 (segment (start 129.335 85.58) (end 121.46 85.58) (width 0.2) (layer "F.Cu") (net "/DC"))
 (segment (start 121.46 85.58) (end 115.54 91.5) (width 0.2) (layer "F.Cu") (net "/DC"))
 (segment (start 118.08 91.5) (end 121.46 88.12) (width 0.2) (layer "F.Cu") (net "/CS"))
 (segment (start 121.46 88.12) (end 128.5 88.12) (width 0.2) (layer "F.Cu") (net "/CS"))
 (segment (start 129.335 88.12) (end 121.46 88.12) (width 0.2) (layer "B.Cu") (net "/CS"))
 (segment (start 121.46 88.12) (end 118.08 91.5) (width 0.2) (layer "B.Cu") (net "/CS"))
 (segment (start 129.335 90.66) (end 121.46 90.66) (width 0.2) (layer "F.Cu") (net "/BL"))
 (segment (start 121.46 90.66) (end 120.62 91.5) (width 0.2) (layer "F.Cu") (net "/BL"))
 (segment (start 111.61 94.340101) (end 106.69 99.260101) (width 0.2) (layer "F.Cu") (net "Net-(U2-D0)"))
 (segment (start 126.58 75.42) (end 111.61 90.39) (width 0.2) (layer "F.Cu") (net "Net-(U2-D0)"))
 (segment (start 106.69 99.260101) (end 106.69 107.33) (width 0.2) (layer "F.Cu") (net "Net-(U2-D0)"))
 (segment (start 129.335 75.42) (end 126.58 75.42) (width 0.2) (layer "F.Cu") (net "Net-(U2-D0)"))
 (segment (start 111.61 90.39) (end 111.61 94.340101) (width 0.2) (layer "F.Cu") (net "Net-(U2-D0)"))
 (segment (start 127.244786 79.438) (end 126.984 79.698786) (width 0.2) (layer "F.Cu") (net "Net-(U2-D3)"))
 (segment (start 136.978895 86.642) (end 129.774895 79.438) (width 0.2) (layer "F.Cu") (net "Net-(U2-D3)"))
 (segment (start 146.665214 81.978) (end 146.926 82.238786) (width 0.2) (layer "F.Cu") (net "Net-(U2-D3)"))
 (segment (start 154.013402 107.33) (end 157.7 103.643402) (width 0.2) (layer "F.Cu") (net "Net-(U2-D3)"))
 (segment (start 129.774895 79.438) (end 127.244786 79.438) (width 0.2) (layer "F.Cu") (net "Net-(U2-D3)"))
 (segment (start 126.984 79.698786) (end 126.984 81.76663) (width 0.2) (layer "F.Cu") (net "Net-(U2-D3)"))
 (segment (start 146.926 82.238786) (end 146.926 86.381214) (width 0.2) (layer "F.Cu") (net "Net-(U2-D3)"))
 (segment (start 157.7 103.643402) (end 157.7 82.861522) (width 0.2) (layer "F.Cu") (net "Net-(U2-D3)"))
 (segment (start 137.642 75.484895) (end 144.135105 81.978) (width 0.2) (layer "F.Cu") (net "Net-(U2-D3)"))
 (segment (start 144.135105 81.978) (end 146.665214 81.978) (width 0.2) (layer "F.Cu") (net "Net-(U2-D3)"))
 (segment (start 137.642 74.358) (end 137.642 75.484895) (width 0.2) (layer "F.Cu") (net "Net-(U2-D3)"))
 (segment (start 146.926 86.381214) (end 146.665214 86.642) (width 0.2) (layer "F.Cu") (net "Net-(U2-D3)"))
 (segment (start 146.665214 86.642) (end 136.978895 86.642) (width 0.2) (layer "F.Cu") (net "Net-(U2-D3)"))
 (segment (start 126.984 81.76663) (end 128.25737 83.04) (width 0.2) (layer "F.Cu") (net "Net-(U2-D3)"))
 (segment (start 149.196478 74.358) (end 137.642 74.358) (width 0.2) (layer "F.Cu") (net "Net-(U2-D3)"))
 (segment (start 157.7 82.861522) (end 149.196478 74.358) (width 0.2) (layer "F.Cu") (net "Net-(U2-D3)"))
 (segment (start 128.25737 83.04) (end 129.335 83.04) (width 0.2) (layer "F.Cu") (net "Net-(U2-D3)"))
 (segment (start 151.96 107.33) (end 154.013402 107.33) (width 0.2) (layer "F.Cu") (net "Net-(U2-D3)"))
 (segment (start 155.94 90.66) (end 156 90.6) (width 0.2) (layer "F.Cu") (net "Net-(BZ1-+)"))
 (segment (start 144.575 90.66) (end 155.94 90.66) (width 0.2) (layer "F.Cu") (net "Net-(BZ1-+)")))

